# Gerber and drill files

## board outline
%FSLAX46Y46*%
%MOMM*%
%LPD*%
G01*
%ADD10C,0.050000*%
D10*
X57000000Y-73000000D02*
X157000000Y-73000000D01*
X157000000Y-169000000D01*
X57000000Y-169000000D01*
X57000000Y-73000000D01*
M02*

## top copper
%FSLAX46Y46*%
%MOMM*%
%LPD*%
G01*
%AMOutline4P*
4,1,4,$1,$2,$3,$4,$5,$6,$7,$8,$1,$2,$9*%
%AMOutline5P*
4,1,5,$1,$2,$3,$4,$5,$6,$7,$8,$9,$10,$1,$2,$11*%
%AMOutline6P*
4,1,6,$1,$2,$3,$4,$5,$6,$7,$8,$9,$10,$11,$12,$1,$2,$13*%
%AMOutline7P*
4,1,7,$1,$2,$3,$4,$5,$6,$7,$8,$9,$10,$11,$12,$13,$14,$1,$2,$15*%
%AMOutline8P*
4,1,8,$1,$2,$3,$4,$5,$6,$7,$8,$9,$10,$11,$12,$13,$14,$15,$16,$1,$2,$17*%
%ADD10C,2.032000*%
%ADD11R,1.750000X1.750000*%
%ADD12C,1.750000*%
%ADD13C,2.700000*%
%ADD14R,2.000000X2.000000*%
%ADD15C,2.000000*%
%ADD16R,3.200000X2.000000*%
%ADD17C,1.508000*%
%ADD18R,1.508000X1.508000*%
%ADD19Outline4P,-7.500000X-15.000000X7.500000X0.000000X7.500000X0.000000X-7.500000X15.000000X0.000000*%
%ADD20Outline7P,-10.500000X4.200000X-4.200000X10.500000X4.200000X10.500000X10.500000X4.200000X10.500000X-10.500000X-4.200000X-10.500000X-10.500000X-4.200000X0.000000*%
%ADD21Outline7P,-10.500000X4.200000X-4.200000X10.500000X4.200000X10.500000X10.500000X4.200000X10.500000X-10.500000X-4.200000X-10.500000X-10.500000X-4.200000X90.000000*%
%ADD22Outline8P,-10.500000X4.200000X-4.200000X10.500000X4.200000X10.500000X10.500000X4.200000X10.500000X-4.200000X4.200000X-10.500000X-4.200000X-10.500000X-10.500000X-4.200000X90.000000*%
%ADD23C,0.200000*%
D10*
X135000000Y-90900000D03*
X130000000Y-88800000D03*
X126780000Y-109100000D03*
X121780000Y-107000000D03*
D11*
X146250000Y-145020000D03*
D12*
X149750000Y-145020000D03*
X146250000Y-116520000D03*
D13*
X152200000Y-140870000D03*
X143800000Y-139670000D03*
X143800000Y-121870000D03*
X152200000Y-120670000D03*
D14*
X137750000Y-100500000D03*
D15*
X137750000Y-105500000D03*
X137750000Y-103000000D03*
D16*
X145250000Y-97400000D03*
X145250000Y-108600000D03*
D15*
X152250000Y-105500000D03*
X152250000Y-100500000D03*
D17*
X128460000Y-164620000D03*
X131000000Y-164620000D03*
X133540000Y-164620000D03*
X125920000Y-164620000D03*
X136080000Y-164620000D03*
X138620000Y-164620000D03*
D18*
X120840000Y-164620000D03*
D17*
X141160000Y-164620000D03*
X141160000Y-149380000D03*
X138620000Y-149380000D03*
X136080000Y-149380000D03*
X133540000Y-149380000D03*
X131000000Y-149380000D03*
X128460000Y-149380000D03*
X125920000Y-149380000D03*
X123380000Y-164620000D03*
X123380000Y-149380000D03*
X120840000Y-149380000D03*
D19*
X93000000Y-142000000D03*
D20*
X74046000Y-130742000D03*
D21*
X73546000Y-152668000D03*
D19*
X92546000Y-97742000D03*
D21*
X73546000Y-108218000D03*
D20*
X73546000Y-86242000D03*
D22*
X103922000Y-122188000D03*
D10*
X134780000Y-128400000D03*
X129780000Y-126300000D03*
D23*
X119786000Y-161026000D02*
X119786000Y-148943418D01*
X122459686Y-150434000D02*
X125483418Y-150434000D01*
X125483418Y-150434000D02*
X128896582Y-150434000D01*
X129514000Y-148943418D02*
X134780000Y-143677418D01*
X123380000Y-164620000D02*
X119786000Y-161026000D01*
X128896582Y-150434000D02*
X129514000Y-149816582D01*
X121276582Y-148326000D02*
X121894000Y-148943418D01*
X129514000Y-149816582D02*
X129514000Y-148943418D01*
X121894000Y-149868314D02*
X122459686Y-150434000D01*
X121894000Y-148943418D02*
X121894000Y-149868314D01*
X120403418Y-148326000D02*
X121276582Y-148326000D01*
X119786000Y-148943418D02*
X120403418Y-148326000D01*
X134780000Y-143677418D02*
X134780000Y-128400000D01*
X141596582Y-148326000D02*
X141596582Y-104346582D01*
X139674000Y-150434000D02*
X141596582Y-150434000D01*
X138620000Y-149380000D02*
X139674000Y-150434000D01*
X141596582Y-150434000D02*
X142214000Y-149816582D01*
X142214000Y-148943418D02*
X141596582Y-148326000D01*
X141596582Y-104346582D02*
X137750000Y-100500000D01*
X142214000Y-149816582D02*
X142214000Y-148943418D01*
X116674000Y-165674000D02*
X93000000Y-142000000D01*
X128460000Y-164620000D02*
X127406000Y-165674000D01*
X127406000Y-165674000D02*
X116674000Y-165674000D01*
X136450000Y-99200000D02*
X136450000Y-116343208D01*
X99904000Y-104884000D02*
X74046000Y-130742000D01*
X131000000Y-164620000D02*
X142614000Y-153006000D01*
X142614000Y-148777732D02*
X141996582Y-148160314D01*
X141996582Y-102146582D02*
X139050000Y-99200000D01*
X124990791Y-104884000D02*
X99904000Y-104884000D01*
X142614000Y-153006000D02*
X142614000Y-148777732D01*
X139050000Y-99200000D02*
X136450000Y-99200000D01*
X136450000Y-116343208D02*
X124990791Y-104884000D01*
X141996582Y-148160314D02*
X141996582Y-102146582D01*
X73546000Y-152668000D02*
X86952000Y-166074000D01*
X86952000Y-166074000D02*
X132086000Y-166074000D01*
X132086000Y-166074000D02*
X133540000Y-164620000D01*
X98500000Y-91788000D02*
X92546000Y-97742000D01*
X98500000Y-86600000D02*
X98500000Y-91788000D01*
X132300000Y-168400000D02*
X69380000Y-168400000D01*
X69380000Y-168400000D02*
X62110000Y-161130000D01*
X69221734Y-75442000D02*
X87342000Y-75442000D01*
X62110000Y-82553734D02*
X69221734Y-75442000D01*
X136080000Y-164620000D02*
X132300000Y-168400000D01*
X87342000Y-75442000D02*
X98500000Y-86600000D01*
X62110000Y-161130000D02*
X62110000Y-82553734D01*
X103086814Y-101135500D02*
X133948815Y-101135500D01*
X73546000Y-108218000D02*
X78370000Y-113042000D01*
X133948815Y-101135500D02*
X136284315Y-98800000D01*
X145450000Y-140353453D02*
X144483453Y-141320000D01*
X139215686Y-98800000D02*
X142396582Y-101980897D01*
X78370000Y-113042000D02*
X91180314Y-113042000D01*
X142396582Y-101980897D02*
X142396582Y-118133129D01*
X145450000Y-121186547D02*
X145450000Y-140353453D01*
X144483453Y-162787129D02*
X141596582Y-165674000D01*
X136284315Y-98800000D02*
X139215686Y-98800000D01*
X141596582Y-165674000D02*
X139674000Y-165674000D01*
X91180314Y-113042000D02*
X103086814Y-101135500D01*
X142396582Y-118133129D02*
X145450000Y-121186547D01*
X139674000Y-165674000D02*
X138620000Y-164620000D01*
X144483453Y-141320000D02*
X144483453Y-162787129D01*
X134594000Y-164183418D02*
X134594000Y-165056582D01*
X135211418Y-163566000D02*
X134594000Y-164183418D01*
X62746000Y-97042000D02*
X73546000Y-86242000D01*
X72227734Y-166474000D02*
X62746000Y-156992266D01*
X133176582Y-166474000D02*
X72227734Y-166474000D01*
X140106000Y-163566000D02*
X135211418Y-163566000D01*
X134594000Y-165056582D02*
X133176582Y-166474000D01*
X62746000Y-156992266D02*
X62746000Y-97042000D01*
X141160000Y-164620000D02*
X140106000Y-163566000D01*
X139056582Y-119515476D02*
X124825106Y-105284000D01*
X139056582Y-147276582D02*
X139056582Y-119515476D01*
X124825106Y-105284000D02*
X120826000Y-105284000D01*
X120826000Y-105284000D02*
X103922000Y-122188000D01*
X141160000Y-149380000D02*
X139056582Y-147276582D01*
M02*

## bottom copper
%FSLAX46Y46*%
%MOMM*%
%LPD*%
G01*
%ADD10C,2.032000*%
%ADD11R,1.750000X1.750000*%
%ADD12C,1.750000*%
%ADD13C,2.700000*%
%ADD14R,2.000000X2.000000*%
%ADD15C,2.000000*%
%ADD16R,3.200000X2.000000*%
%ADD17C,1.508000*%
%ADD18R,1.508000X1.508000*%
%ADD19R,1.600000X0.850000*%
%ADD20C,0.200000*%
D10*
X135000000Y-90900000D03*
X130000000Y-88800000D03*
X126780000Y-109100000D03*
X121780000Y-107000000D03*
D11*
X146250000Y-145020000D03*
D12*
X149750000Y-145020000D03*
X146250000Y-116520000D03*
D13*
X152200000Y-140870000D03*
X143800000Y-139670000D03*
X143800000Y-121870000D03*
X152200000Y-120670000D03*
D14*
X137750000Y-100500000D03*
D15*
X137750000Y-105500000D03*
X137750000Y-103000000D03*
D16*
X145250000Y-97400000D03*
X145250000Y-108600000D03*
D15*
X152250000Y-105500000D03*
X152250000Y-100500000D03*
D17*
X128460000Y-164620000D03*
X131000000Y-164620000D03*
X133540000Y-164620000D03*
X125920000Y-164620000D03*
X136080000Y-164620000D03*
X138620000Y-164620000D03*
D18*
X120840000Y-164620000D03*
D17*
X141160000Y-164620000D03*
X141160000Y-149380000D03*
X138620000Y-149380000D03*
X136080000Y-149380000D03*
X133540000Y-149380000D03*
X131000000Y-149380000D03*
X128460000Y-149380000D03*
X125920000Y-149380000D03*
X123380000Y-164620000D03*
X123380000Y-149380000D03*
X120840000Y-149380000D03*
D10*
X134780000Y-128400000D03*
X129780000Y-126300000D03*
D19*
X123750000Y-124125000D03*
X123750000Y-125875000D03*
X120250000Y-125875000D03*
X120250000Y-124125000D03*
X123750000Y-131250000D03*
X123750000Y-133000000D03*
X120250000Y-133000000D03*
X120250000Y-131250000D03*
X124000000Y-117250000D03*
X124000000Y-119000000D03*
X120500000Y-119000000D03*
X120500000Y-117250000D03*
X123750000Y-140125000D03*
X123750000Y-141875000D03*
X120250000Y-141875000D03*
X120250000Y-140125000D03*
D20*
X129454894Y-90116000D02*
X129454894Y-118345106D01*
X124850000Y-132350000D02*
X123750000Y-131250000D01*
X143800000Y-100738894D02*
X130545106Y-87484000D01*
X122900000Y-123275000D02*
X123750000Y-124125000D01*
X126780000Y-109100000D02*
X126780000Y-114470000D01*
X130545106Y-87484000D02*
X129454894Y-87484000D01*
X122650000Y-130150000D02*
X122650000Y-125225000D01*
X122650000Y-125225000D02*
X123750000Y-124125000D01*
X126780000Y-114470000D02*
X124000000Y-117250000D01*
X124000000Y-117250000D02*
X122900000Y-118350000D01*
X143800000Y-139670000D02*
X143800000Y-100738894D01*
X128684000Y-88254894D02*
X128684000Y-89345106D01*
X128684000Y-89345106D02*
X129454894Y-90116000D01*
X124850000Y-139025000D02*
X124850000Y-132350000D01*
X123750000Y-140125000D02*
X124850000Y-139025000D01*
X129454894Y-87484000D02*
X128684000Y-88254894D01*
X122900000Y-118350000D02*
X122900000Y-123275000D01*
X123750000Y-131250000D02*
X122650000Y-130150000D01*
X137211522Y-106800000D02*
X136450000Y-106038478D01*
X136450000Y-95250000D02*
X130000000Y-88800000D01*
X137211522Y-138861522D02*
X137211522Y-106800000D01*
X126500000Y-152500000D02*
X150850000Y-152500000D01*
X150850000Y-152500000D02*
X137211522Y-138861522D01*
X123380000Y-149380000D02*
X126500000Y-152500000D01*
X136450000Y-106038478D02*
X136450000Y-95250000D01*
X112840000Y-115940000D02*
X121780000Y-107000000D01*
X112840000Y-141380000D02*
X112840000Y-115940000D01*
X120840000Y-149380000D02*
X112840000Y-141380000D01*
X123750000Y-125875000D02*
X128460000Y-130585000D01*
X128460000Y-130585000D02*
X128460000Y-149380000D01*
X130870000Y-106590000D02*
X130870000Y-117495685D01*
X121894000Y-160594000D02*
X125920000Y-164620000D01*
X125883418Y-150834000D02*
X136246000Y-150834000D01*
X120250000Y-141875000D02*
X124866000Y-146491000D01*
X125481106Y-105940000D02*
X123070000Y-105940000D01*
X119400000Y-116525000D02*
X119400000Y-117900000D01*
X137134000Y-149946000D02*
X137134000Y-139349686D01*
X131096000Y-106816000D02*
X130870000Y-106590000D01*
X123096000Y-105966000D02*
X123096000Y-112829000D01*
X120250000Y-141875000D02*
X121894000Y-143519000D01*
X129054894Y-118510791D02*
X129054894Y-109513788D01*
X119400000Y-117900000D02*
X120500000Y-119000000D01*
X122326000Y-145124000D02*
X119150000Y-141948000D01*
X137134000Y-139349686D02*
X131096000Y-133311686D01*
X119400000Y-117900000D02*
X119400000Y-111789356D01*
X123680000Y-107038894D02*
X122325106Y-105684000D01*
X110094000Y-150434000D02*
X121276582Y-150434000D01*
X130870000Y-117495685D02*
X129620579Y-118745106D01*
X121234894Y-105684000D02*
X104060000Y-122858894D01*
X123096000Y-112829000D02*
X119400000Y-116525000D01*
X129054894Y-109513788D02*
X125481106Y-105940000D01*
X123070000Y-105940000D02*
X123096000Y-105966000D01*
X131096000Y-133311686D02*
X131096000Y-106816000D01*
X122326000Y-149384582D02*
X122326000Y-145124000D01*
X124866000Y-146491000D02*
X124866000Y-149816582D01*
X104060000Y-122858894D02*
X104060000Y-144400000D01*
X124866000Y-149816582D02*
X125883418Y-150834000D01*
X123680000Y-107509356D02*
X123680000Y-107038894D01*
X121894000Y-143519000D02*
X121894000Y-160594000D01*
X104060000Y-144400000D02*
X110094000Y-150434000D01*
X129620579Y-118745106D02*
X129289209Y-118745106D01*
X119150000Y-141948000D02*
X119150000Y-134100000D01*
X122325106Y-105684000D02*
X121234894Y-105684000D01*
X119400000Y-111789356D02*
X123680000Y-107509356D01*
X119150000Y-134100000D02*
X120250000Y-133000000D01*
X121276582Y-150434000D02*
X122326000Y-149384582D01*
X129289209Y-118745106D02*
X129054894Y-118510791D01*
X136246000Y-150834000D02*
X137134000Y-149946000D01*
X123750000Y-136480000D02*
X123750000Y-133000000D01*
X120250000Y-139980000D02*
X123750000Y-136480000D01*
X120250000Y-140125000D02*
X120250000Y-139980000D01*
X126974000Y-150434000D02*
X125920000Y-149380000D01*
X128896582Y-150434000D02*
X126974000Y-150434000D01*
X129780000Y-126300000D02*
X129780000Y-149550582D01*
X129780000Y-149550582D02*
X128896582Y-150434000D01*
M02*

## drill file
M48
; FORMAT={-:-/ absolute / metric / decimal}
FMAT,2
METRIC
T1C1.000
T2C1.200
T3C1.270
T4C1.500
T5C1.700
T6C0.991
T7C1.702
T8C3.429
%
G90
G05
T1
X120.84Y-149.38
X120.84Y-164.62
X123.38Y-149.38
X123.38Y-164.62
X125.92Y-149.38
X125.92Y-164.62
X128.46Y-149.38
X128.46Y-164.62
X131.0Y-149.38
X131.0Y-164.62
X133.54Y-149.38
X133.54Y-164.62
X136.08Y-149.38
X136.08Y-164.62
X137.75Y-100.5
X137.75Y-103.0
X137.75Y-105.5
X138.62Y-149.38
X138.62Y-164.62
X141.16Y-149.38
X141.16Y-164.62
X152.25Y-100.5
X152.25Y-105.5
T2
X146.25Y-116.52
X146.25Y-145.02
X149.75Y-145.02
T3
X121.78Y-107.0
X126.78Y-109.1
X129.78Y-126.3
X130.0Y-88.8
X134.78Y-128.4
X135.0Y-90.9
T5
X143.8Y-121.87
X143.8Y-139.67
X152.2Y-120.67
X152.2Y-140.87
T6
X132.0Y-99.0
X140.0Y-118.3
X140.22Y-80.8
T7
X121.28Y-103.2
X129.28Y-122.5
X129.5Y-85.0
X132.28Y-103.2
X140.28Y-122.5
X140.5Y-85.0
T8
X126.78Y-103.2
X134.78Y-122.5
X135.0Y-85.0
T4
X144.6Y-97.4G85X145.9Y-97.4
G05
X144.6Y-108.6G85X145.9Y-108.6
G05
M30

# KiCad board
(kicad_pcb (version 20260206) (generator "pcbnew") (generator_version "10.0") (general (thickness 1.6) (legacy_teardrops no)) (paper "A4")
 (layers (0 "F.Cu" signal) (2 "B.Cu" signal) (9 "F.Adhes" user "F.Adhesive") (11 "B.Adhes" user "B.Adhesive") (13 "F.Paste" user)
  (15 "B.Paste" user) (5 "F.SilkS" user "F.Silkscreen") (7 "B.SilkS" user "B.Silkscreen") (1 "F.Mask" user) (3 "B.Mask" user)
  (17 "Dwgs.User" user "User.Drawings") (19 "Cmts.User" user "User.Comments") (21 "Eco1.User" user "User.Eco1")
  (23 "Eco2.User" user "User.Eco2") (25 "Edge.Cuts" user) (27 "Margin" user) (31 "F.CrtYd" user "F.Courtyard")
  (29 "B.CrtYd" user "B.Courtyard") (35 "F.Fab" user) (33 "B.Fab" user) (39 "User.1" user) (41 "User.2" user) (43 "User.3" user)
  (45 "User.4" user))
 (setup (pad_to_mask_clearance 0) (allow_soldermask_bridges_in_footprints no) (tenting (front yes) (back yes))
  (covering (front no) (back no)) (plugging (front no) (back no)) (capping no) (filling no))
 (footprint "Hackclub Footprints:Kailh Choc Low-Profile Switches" (layer "F.Cu") (at 135 85)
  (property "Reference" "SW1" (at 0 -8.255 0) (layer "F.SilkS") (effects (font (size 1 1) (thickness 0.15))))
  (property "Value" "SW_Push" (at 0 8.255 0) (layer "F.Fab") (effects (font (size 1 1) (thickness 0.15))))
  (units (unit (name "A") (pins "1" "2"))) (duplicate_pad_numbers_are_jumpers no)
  (pad "" np_thru_hole circle (at -5.5 0) (size 1.7018 1.7018) (drill 1.7018) (layers "*.Cu" "*.Mask"))
  (pad "" np_thru_hole circle (at 0 0) (size 3.429 3.429) (drill 3.429) (layers "*.Cu" "*.Mask"))
  (pad "" np_thru_hole circle (at 5.22 -4.2) (size 0.9906 0.9906) (drill 0.9906) (layers "*.Cu" "*.Mask"))
  (pad "" np_thru_hole circle (at 5.5 0) (size 1.7018 1.7018) (drill 1.7018) (layers "*.Cu" "*.Mask"))
  (pad "1" thru_hole circle (at 0 5.9) (size 2.032 2.032) (drill 1.27) (layers "*.Cu" "*.Mask") (remove_unused_layers no) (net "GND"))
  (pad "2" thru_hole circle (at -5 3.8) (size 2.032 2.032) (drill 1.27) (layers "*.Cu" "*.Mask") (remove_unused_layers no) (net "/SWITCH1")))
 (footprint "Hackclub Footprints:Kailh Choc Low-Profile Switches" (layer "F.Cu") (at 126.78 103.2)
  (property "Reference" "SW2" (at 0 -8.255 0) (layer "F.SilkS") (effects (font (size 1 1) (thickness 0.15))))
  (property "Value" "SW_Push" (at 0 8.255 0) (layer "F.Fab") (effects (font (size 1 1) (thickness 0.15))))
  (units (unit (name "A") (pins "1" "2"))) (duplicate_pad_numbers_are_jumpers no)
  (pad "" np_thru_hole circle (at -5.5 0) (size 1.7018 1.7018) (drill 1.7018) (layers "*.Cu" "*.Mask"))
  (pad "" np_thru_hole circle (at 0 0) (size 3.429 3.429) (drill 3.429) (layers "*.Cu" "*.Mask"))
  (pad "" np_thru_hole circle (at 5.22 -4.2) (size 0.9906 0.9906) (drill 0.9906) (layers "*.Cu" "*.Mask"))
  (pad "" np_thru_hole circle (at 5.5 0) (size 1.7018 1.7018) (drill 1.7018) (layers "*.Cu" "*.Mask"))
  (pad "1" thru_hole circle (at 0 5.9) (size 2.032 2.032) (drill 1.27) (layers "*.Cu" "*.Mask") (remove_unused_layers no) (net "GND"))
  (pad "2" thru_hole circle (at -5 3.8) (size 2.032 2.032) (drill 1.27) (layers "*.Cu" "*.Mask") (remove_unused_layers no) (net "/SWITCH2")))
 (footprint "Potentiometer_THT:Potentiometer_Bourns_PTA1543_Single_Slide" (layer "F.Cu") (at 146.25 145.02 90)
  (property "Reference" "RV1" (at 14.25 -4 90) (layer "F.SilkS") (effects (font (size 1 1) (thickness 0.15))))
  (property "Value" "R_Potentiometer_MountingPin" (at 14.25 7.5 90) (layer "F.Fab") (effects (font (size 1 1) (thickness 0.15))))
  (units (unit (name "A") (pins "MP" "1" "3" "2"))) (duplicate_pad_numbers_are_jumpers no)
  (pad "1" thru_hole rect (at 0 0 90) (size 1.75 1.75) (drill 1.2) (layers "*.Cu" "*.Mask") (remove_unused_layers no)
   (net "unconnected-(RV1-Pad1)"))
  (pad "2" thru_hole circle (at 0 3.5 90) (size 1.75 1.75) (drill 1.2) (layers "*.Cu" "*.Mask") (remove_unused_layers no) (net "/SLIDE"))
  (pad "3" thru_hole circle (at 28.5 0 90) (size 1.75 1.75) (drill 1.2) (layers "*.Cu" "*.Mask") (remove_unused_layers no) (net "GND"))
  (pad "MP" thru_hole circle (at 4.15 5.95 90) (size 2.7 2.7) (drill 1.7) (layers "*.Cu" "*.Mask") (remove_unused_layers no) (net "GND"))
  (pad "MP" thru_hole circle (at 5.35 -2.45 90) (size 2.7 2.7) (drill 1.7) (layers "*.Cu" "*.Mask") (remove_unused_layers no) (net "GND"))
  (pad "MP" thru_hole circle (at 23.15 -2.45 90) (size 2.7 2.7) (drill 1.7) (layers "*.Cu" "*.Mask") (remove_unused_layers no) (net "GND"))
  (pad "MP" thru_hole circle (at 24.35 5.95 90) (size 2.7 2.7) (drill 1.7) (layers "*.Cu" "*.Mask") (remove_unused_layers no) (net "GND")))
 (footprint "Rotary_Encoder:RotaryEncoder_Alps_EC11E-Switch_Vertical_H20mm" (layer "F.Cu") (at 137.75 100.5)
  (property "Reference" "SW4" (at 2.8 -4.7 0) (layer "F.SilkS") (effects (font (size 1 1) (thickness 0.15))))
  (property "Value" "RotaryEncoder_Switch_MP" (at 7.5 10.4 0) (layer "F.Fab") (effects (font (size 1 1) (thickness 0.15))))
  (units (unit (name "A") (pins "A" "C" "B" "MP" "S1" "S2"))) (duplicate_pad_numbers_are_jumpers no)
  (pad "A" thru_hole rect (at 0 0) (size 2 2) (drill 1) (layers "*.Cu" "*.Mask") (remove_unused_layers no) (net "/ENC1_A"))
  (pad "B" thru_hole circle (at 0 5) (size 2 2) (drill 1) (layers "*.Cu" "*.Mask") (remove_unused_layers no) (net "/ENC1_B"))
  (pad "C" thru_hole circle (at 0 2.5) (size 2 2) (drill 1) (layers "*.Cu" "*.Mask") (remove_unused_layers no) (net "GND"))
  (pad "MP" thru_hole rect (at 7.5 -3.1) (size 3.2 2) (drill oval 2.8 1.5) (layers "*.Cu" "*.Mask") (remove_unused_layers no) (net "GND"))
  (pad "MP" thru_hole rect (at 7.5 8.1) (size 3.2 2) (drill oval 2.8 1.5) (layers "*.Cu" "*.Mask") (remove_unused_layers no) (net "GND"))
  (pad "S1" thru_hole circle (at 14.5 5) (size 2 2) (drill 1) (layers "*.Cu" "*.Mask") (remove_unused_layers no) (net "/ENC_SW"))
  (pad "S2" thru_hole circle (at 14.5 0) (size 2 2) (drill 1) (layers "*.Cu" "*.Mask") (remove_unused_layers no)
   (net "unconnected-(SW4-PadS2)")))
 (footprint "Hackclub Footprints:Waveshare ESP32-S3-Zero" (layer "F.Cu") (at 131 157 90)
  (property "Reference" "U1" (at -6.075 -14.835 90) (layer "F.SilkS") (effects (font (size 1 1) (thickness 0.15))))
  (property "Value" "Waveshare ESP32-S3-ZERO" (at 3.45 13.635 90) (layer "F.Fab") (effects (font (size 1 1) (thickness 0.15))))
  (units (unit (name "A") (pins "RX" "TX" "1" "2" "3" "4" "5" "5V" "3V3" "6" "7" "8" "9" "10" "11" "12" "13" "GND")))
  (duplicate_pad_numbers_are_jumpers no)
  (pad "1" thru_hole circle (at -7.62 -2.54 90) (size 1.508 1.508) (drill 1) (layers "*.Cu" "*.Mask") (remove_unused_layers no)
   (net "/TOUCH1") (solder_mask_margin 0.102))
  (pad "2" thru_hole circle (at -7.62 0 90) (size 1.508 1.508) (drill 1) (layers "*.Cu" "*.Mask") (remove_unused_layers no) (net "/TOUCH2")
   (solder_mask_margin 0.102))
  (pad "3" thru_hole circle (at -7.62 2.54 90) (size 1.508 1.508) (drill 1) (layers "*.Cu" "*.Mask") (remove_unused_layers no)
   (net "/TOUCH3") (solder_mask_margin 0.102))
  (pad "3V3" thru_hole circle (at -7.62 -5.08 90) (size 1.508 1.508) (drill 1) (layers "*.Cu" "*.Mask") (remove_unused_layers no)
   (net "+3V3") (solder_mask_margin 0.102))
  (pad "4" thru_hole circle (at -7.62 5.08 90) (size 1.508 1.508) (drill 1) (layers "*.Cu" "*.Mask") (remove_unused_layers no)
   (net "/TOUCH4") (solder_mask_margin 0.102))
  (pad "5" thru_hole circle (at -7.62 7.62 90) (size 1.508 1.508) (drill 1) (layers "*.Cu" "*.Mask") (remove_unused_layers no)
   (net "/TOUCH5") (solder_mask_margin 0.102))
  (pad "5V" thru_hole rect (at -7.62 -10.16 90) (size 1.508 1.508) (drill 1) (layers "*.Cu" "*.Mask") (remove_unused_layers no) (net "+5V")
   (solder_mask_margin 0.102))
  (pad "6" thru_hole circle (at -7.62 10.16 90) (size 1.508 1.508) (drill 1) (layers "*.Cu" "*.Mask") (remove_unused_layers no)
   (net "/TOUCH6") (solder_mask_margin 0.102))
  (pad "7" thru_hole circle (at 7.62 10.16 90) (size 1.508 1.508) (drill 1) (layers "*.Cu" "*.Mask") (remove_unused_layers no)
   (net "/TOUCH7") (solder_mask_margin 0.102))
  (pad "8" thru_hole circle (at 7.62 7.62 90) (size 1.508 1.508) (drill 1) (layers "*.Cu" "*.Mask") (remove_unused_layers no)
   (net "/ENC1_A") (solder_mask_margin 0.102))
  (pad "9" thru_hole circle (at 7.62 5.08 90) (size 1.508 1.508) (drill 1) (layers "*.Cu" "*.Mask") (remove_unused_layers no)
   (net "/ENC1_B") (solder_mask_margin 0.102))
  (pad "10" thru_hole circle (at 7.62 2.54 90) (size 1.508 1.508) (drill 1) (layers "*.Cu" "*.Mask") (remove_unused_layers no)
   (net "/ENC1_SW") (solder_mask_margin 0.102))
  (pad "11" thru_hole circle (at 7.62 0 90) (size 1.508 1.508) (drill 1) (layers "*.Cu" "*.Mask") (remove_unused_layers no) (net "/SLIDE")
   (solder_mask_margin 0.102))
  (pad "12" thru_hole circle (at 7.62 -2.54 90) (size 1.508 1.508) (drill 1) (layers "*.Cu" "*.Mask") (remove_unused_layers no) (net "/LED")
   (solder_mask_margin 0.102))
  (pad "13" thru_hole circle (at 7.62 -5.08 90) (size 1.508 1.508) (drill 1) (layers "*.Cu" "*.Mask") (remove_unused_layers no)
   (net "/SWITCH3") (solder_mask_margin 0.102))
  (pad "GND" thru_hole circle (at -7.62 -7.62 90) (size 1.508 1.508) (drill 1) (layers "*.Cu" "*.Mask") (remove_unused_layers no)
   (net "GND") (solder_mask_margin 0.102))
  (pad "RX" thru_hole circle (at 7.62 -7.62 90) (size 1.508 1.508) (drill 1) (layers "*.Cu" "*.Mask") (remove_unused_layers no)
   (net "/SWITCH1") (solder_mask_margin 0.102))
  (pad "TX" thru_hole circle (at 7.62 -10.16 90) (size 1.508 1.508) (drill 1) (layers "*.Cu" "*.Mask") (remove_unused_layers no)
   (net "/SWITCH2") (solder_mask_margin 0.102)))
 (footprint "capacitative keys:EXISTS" (layer "F.Cu") (at 80.046 109.742)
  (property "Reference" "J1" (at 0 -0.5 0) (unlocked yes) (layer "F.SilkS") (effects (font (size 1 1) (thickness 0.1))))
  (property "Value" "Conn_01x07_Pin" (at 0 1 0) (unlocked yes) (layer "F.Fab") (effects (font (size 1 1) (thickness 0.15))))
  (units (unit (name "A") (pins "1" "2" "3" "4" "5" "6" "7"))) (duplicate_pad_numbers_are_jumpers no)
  (pad "1" smd trapezoid (at 12.954 32.258) (size 15 15) (rect_delta 15 0) (layers "F.Cu" "F.Mask") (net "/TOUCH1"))
  (pad "2" smd roundrect (at -6 21) (size 21 21) (layers "F.Cu" "F.Mask") (roundrect_rratio 0) (chamfer_ratio 0.3)
   (chamfer top_left top_right bottom_left) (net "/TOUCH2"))
  (pad "3" smd roundrect (at -6.5 42.926 90) (size 21 21) (layers "F.Cu" "F.Mask") (roundrect_rratio 0) (chamfer_ratio 0.3)
   (chamfer top_left top_right bottom_left) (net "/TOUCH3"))
  (pad "4" smd trapezoid (at 12.5 -12) (size 15 15) (rect_delta 15 0) (layers "F.Cu" "F.Mask") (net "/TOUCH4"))
  (pad "5" smd roundrect (at -6.5 -1.524 90) (size 21 21) (layers "F.Cu" "F.Mask") (roundrect_rratio 0) (chamfer_ratio 0.3)
   (chamfer top_left top_right bottom_left) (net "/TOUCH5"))
  (pad "6" smd roundrect (at -6.5 -23.5) (size 21 21) (layers "F.Cu" "F.Mask") (roundrect_rratio 0) (chamfer_ratio 0.3)
   (chamfer top_left top_right bottom_left) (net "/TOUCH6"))
  (pad "7" smd roundrect (at 23.876 12.446 90) (size 21 21) (layers "F.Cu" "F.Mask") (roundrect_rratio 0) (chamfer_ratio 0.3)
   (chamfer top_left top_right bottom_left bottom_right) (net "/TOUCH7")))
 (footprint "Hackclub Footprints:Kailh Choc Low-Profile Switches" (layer "F.Cu") (at 134.78 122.5)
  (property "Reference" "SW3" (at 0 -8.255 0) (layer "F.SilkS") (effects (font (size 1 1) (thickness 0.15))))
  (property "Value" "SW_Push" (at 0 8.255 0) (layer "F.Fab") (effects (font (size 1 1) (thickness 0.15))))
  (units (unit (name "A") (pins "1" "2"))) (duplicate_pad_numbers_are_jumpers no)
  (pad "" np_thru_hole circle (at -5.5 0) (size 1.7018 1.7018) (drill 1.7018) (layers "*.Cu" "*.Mask"))
  (pad "" np_thru_hole circle (at 0 0) (size 3.429 3.429) (drill 3.429) (layers "*.Cu" "*.Mask"))
  (pad "" np_thru_hole circle (at 5.22 -4.2) (size 0.9906 0.9906) (drill 0.9906) (layers "*.Cu" "*.Mask"))
  (pad "" np_thru_hole circle (at 5.5 0) (size 1.7018 1.7018) (drill 1.7018) (layers "*.Cu" "*.Mask"))
  (pad "1" thru_hole circle (at 0 5.9) (size 2.032 2.032) (drill 1.27) (layers "*.Cu" "*.Mask") (remove_unused_layers no) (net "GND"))
  (pad "2" thru_hole circle (at -5 3.8) (size 2.032 2.032) (drill 1.27) (layers "*.Cu" "*.Mask") (remove_unused_layers no) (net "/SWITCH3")))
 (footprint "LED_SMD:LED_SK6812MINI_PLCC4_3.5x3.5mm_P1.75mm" (layer "B.Cu") (at 122 125 180)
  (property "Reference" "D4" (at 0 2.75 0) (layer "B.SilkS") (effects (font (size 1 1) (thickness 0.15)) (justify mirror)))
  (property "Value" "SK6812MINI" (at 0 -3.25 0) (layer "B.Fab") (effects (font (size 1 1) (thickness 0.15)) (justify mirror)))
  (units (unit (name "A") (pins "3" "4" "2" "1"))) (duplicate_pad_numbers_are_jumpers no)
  (pad "1" smd rect (at -1.75 0.875 180) (size 1.6 0.85) (layers "B.Cu" "B.Mask" "B.Paste") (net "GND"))
  (pad "2" smd rect (at -1.75 -0.875 180) (size 1.6 0.85) (layers "B.Cu" "B.Mask" "B.Paste") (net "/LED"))
  (pad "3" smd rect (at 1.75 -0.875 180) (size 1.6 0.85) (layers "B.Cu" "B.Mask" "B.Paste") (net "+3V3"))
  (pad "4" smd rect (at 1.75 0.875 180) (size 1.6 0.85) (layers "B.Cu" "B.Mask" "B.Paste") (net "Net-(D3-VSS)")))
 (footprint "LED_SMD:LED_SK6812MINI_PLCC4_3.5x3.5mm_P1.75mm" (layer "B.Cu") (at 122 132.125 180)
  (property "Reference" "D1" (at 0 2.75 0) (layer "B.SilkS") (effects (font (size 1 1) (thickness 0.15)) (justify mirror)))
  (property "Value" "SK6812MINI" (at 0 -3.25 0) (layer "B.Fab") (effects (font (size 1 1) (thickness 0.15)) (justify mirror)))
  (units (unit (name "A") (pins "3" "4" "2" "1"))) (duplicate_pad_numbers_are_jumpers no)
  (pad "1" smd rect (at -1.75 0.875 180) (size 1.6 0.85) (layers "B.Cu" "B.Mask" "B.Paste") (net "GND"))
  (pad "2" smd rect (at -1.75 -0.875 180) (size 1.6 0.85) (layers "B.Cu" "B.Mask" "B.Paste") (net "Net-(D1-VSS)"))
  (pad "3" smd rect (at 1.75 -0.875 180) (size 1.6 0.85) (layers "B.Cu" "B.Mask" "B.Paste") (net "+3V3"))
  (pad "4" smd rect (at 1.75 0.875 180) (size 1.6 0.85) (layers "B.Cu" "B.Mask" "B.Paste") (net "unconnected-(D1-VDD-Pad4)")))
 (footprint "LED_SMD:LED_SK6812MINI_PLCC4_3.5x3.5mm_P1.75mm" (layer "B.Cu") (at 122.25 118.125 180)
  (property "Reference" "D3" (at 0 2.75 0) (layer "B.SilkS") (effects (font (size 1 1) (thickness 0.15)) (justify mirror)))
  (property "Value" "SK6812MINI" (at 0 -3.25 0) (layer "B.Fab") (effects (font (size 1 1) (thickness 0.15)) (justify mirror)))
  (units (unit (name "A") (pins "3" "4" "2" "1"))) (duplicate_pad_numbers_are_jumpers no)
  (pad "1" smd rect (at -1.75 0.875 180) (size 1.6 0.85) (layers "B.Cu" "B.Mask" "B.Paste") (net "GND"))
  (pad "2" smd rect (at -1.75 -0.875 180) (size 1.6 0.85) (layers "B.Cu" "B.Mask" "B.Paste") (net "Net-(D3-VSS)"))
  (pad "3" smd rect (at 1.75 -0.875 180) (size 1.6 0.85) (layers "B.Cu" "B.Mask" "B.Paste") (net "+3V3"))
  (pad "4" smd rect (at 1.75 0.875 180) (size 1.6 0.85) (layers "B.Cu" "B.Mask" "B.Paste") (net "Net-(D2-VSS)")))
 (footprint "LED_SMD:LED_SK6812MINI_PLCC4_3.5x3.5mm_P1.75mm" (layer "B.Cu") (at 122 141 180)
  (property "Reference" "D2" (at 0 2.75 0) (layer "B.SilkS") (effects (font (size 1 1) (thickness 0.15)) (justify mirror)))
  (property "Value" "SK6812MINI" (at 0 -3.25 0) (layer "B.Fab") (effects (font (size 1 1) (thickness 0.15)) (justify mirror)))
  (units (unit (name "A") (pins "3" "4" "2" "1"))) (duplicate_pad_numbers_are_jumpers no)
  (pad "1" smd rect (at -1.75 0.875 180) (size 1.6 0.85) (layers "B.Cu" "B.Mask" "B.Paste") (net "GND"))
  (pad "2" smd rect (at -1.75 -0.875 180) (size 1.6 0.85) (layers "B.Cu" "B.Mask" "B.Paste") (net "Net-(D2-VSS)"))
  (pad "3" smd rect (at 1.75 -0.875 180) (size 1.6 0.85) (layers "B.Cu" "B.Mask" "B.Paste") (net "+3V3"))
  (pad "4" smd rect (at 1.75 0.875 180) (size 1.6 0.85) (layers "B.Cu" "B.Mask" "B.Paste") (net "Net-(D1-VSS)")))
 (gr_rect (start 57 73) (end 157 169) (stroke (width 0.05) (type default)) (fill no) (layer "Edge.Cuts"))
 (segment (start 119.786 161.026) (end 119.786 148.943418) (width 0.2) (layer "F.Cu") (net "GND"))
 (segment (start 122.459686 150.434) (end 125.483418 150.434) (width 0.2) (layer "F.Cu") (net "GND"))
 (segment (start 125.483418 150.434) (end 128.896582 150.434) (width 0.2) (layer "F.Cu") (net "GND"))
 (segment (start 129.514 148.943418) (end 134.78 143.677418) (width 0.2) (layer "F.Cu") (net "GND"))
 (segment (start 123.38 164.62) (end 119.786 161.026) (width 0.2) (layer "F.Cu") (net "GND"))
 (segment (start 128.896582 150.434) (end 129.514 149.816582) (width 0.2) (layer "F.Cu") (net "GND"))
 (segment (start 121.276582 148.326) (end 121.894 148.943418) (width 0.2) (layer "F.Cu") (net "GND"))
 (segment (start 129.514 149.816582) (end 129.514 148.943418) (width 0.2) (layer "F.Cu") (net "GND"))
 (segment (start 121.894 149.868314) (end 122.459686 150.434) (width 0.2) (layer "F.Cu") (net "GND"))
 (segment (start 121.894 148.943418) (end 121.894 149.868314) (width 0.2) (layer "F.Cu") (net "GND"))
 (segment (start 120.403418 148.326) (end 121.276582 148.326) (width 0.2) (layer "F.Cu") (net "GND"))
 (segment (start 119.786 148.943418) (end 120.403418 148.326) (width 0.2) (layer "F.Cu") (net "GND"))
 (segment (start 134.78 143.677418) (end 134.78 128.4) (width 0.2) (layer "F.Cu") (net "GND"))
 (segment (start 129.454894 90.116) (end 129.454894 118.345106) (width 0.2) (layer "B.Cu") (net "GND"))
 (segment (start 124.85 132.35) (end 123.75 131.25) (width 0.2) (layer "B.Cu") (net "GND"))
 (segment (start 143.8 100.738894) (end 130.545106 87.484) (width 0.2) (layer "B.Cu") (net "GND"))
 (segment (start 122.9 123.275) (end 123.75 124.125) (width 0.2) (layer "B.Cu") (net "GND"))
 (segment (start 126.78 109.1) (end 126.78 114.47) (width 0.2) (layer "B.Cu") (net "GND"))
 (segment (start 130.545106 87.484) (end 129.454894 87.484) (width 0.2) (layer "B.Cu") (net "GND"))
 (segment (start 122.65 130.15) (end 122.65 125.225) (width 0.2) (layer "B.Cu") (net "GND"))
 (segment (start 122.65 125.225) (end 123.75 124.125) (width 0.2) (layer "B.Cu") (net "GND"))
 (segment (start 126.78 114.47) (end 124 117.25) (width 0.2) (layer "B.Cu") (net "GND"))
 (segment (start 124 117.25) (end 122.9 118.35) (width 0.2) (layer "B.Cu") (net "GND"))
 (segment (start 143.8 139.67) (end 143.8 100.738894) (width 0.2) (layer "B.Cu") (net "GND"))
 (segment (start 128.684 88.254894) (end 128.684 89.345106) (width 0.2) (layer "B.Cu") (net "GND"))
 (segment (start 128.684 89.345106) (end 129.454894 90.116) (width 0.2) (layer "B.Cu") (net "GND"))
 (segment (start 124.85 139.025) (end 124.85 132.35) (width 0.2) (layer "B.Cu") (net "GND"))
 (segment (start 123.75 140.125) (end 124.85 139.025) (width 0.2) (layer "B.Cu") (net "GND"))
 (segment (start 129.454894 87.484) (end 128.684 88.254894) (width 0.2) (layer "B.Cu") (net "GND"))
 (segment (start 122.9 118.35) (end 122.9 123.275) (width 0.2) (layer "B.Cu") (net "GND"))
 (segment (start 123.75 131.25) (end 122.65 130.15) (width 0.2) (layer "B.Cu") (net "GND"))
 (segment (start 137.211522 106.8) (end 136.45 106.038478) (width 0.2) (layer "B.Cu") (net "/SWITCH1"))
 (segment (start 136.45 95.25) (end 130 88.8) (width 0.2) (layer "B.Cu") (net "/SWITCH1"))
 (segment (start 137.211522 138.861522) (end 137.211522 106.8) (width 0.2) (layer "B.Cu") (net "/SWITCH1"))
 (segment (start 126.5 152.5) (end 150.85 152.5) (width 0.2) (layer "B.Cu") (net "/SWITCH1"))
 (segment (start 150.85 152.5) (end 137.211522 138.861522) (width 0.2) (layer "B.Cu") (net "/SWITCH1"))
 (segment (start 123.38 149.38) (end 126.5 152.5) (width 0.2) (layer "B.Cu") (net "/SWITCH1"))
 (segment (start 136.45 106.038478) (end 136.45 95.25) (width 0.2) (layer "B.Cu") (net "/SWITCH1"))
 (segment (start 112.84 115.94) (end 121.78 107) (width 0.2) (layer "B.Cu") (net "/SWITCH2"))
 (segment (start 112.84 141.38) (end 112.84 115.94) (width 0.2) (layer "B.Cu") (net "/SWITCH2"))
 (segment (start 120.84 149.38) (end 112.84 141.38) (width 0.2) (layer "B.Cu") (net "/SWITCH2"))
 (segment (start 123.75 125.875) (end 128.46 130.585) (width 0.2) (layer "B.Cu") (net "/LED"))
 (segment (start 128.46 130.585) (end 128.46 149.38) (width 0.2) (layer "B.Cu") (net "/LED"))
 (segment (start 130.87 106.59) (end 130.87 117.495685) (width 0.2) (layer "B.Cu") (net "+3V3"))
 (segment (start 121.894 160.594) (end 125.92 164.62) (width 0.2) (layer "B.Cu") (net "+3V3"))
 (segment (start 125.883418 150.834) (end 136.246 150.834) (width 0.2) (layer "B.Cu") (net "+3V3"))
 (segment (start 120.25 141.875) (end 124.866 146.491) (width 0.2) (layer "B.Cu") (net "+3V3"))
 (segment (start 125.481106 105.94) (end 123.07 105.94) (width 0.2) (layer "B.Cu") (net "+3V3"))
 (segment (start 119.4 116.525) (end 119.4 117.9) (width 0.2) (layer "B.Cu") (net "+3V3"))
 (segment (start 137.134 149.946) (end 137.134 139.349686) (width 0.2) (layer "B.Cu") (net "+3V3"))
 (segment (start 131.096 106.816) (end 130.87 106.59) (width 0.2) (layer "B.Cu") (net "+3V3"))
 (segment (start 123.096 105.966) (end 123.096 112.829) (width 0.2) (layer "B.Cu") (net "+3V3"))
 (segment (start 120.25 141.875) (end 121.894 143.519) (width 0.2) (layer "B.Cu") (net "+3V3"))
 (segment (start 129.054894 118.510791) (end 129.054894 109.513788) (width 0.2) (layer "B.Cu") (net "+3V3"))
 (segment (start 119.4 117.9) (end 120.5 119) (width 0.2) (layer "B.Cu") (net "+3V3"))
 (segment (start 122.326 145.124) (end 119.15 141.948) (width 0.2) (layer "B.Cu") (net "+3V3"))
 (segment (start 137.134 139.349686) (end 131.096 133.311686) (width 0.2) (layer "B.Cu") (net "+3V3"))
 (segment (start 119.4 117.9) (end 119.4 111.789356) (width 0.2) (layer "B.Cu") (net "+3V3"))
 (segment (start 123.68 107.038894) (end 122.325106 105.684) (width 0.2) (layer "B.Cu") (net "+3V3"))
 (segment (start 110.094 150.434) (end 121.276582 150.434) (width 0.2) (layer "B.Cu") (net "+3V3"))
 (segment (start 130.87 117.495685) (end 129.620579 118.745106) (width 0.2) (layer "B.Cu") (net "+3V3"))
 (segment (start 121.234894 105.684) (end 104.06 122.858894) (width 0.2) (layer "B.Cu") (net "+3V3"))
 (segment (start 123.096 112.829) (end 119.4 116.525) (width 0.2) (layer "B.Cu") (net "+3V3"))
 (segment (start 129.054894 109.513788) (end 125.481106 105.94) (width 0.2) (layer "B.Cu") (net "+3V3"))
 (segment (start 123.07 105.94) (end 123.096 105.966) (width 0.2) (layer "B.Cu") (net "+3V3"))
 (segment (start 131.096 133.311686) (end 131.096 106.816) (width 0.2) (layer "B.Cu") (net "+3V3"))
 (segment (start 122.326 149.384582) (end 122.326 145.124) (width 0.2) (layer "B.Cu") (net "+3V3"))
 (segment (start 124.866 146.491) (end 124.866 149.816582) (width 0.2) (layer "B.Cu") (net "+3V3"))
 (segment (start 104.06 122.858894) (end 104.06 144.4) (width 0.2) (layer "B.Cu") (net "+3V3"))
 (segment (start 124.866 149.816582) (end 125.883418 150.834) (width 0.2) (layer "B.Cu") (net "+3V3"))
 (segment (start 123.68 107.509356) (end 123.68 107.038894) (width 0.2) (layer "B.Cu") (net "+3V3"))
 (segment (start 121.894 143.519) (end 121.894 160.594) (width 0.2) (layer "B.Cu") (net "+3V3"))
 (segment (start 104.06 144.4) (end 110.094 150.434) (width 0.2) (layer "B.Cu") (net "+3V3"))
 (segment (start 129.620579 118.745106) (end 129.289209 118.745106) (width 0.2) (layer "B.Cu") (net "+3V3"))
 (segment (start 119.15 141.948) (end 119.15 134.1) (width 0.2) (layer "B.Cu") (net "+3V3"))
 (segment (start 122.325106 105.684) (end 121.234894 105.684) (width 0.2) (layer "B.Cu") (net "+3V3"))
 (segment (start 119.4 111.789356) (end 123.68 107.509356) (width 0.2) (layer "B.Cu") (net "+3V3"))
 (segment (start 119.15 134.1) (end 120.25 133) (width 0.2) (layer "B.Cu") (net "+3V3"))
 (segment (start 121.276582 150.434) (end 122.326 149.384582) (width 0.2) (layer "B.Cu") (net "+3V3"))
 (segment (start 129.289209 118.745106) (end 129.054894 118.510791) (width 0.2) (layer "B.Cu") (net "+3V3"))
 (segment (start 136.246 150.834) (end 137.134 149.946) (width 0.2) (layer "B.Cu") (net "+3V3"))
 (segment (start 141.596582 148.326) (end 141.596582 104.346582) (width 0.2) (layer "F.Cu") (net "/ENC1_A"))
 (segment (start 139.674 150.434) (end 141.596582 150.434) (width 0.2) (layer "F.Cu") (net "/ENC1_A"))
 (segment (start 138.62 149.38) (end 139.674 150.434) (width 0.2) (layer "F.Cu") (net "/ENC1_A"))
 (segment (start 141.596582 150.434) (end 142.214 149.816582) (width 0.2) (layer "F.Cu") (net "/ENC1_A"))
 (segment (start 142.214 148.943418) (end 141.596582 148.326) (width 0.2) (layer "F.Cu") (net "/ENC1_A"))
 (segment (start 141.596582 104.346582) (end 137.75 100.5) (width 0.2) (layer "F.Cu") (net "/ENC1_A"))
 (segment (start 142.214 149.816582) (end 142.214 148.943418) (width 0.2) (layer "F.Cu") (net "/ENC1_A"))
 (segment (start 123.75 136.48) (end 123.75 133) (width 0.2) (layer "B.Cu") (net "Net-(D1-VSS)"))
 (segment (start 120.25 139.98) (end 123.75 136.48) (width 0.2) (layer "B.Cu") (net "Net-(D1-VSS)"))
 (segment (start 120.25 140.125) (end 120.25 139.98) (width 0.2) (layer "B.Cu") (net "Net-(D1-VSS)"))
 (segment (start 116.674 165.674) (end 93 142) (width 0.2) (layer "F.Cu") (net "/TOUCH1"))
 (segment (start 128.46 164.62) (end 127.406 165.674) (width 0.2) (layer "F.Cu") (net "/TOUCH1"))
 (segment (start 127.406 165.674) (end 116.674 165.674) (width 0.2) (layer "F.Cu") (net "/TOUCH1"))
 (segment (start 136.45 99.2) (end 136.45 116.343208) (width 0.2) (layer "F.Cu") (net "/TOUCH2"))
 (segment (start 99.904 104.884) (end 74.046 130.742) (width 0.2) (layer "F.Cu") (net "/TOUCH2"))
 (segment (start 131 164.62) (end 142.614 153.006) (width 0.2) (layer "F.Cu") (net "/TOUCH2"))
 (segment (start 142.614 148.777732) (end 141.996582 148.160314) (width 0.2) (layer "F.Cu") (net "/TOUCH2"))
 (segment (start 141.996582 102.146582) (end 139.05 99.2) (width 0.2) (layer "F.Cu") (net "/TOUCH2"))
 (segment (start 124.990791 104.884) (end 99.904 104.884) (width 0.2) (layer "F.Cu") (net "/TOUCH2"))
 (segment (start 142.614 153.006) (end 142.614 148.777732) (width 0.2) (layer "F.Cu") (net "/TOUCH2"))
 (segment (start 139.05 99.2) (end 136.45 99.2) (width 0.2) (layer "F.Cu") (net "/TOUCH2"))
 (segment (start 136.45 116.343208) (end 124.990791 104.884) (width 0.2) (layer "F.Cu") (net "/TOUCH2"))
 (segment (start 141.996582 148.160314) (end 141.996582 102.146582) (width 0.2) (layer "F.Cu") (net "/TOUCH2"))
 (segment (start 73.546 152.668) (end 86.952 166.074) (width 0.2) (layer "F.Cu") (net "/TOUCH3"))
 (segment (start 86.952 166.074) (end 132.086 166.074) (width 0.2) (layer "F.Cu") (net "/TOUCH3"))
 (segment (start 132.086 166.074) (end 133.54 164.62) (width 0.2) (layer "F.Cu") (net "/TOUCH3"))
 (segment (start 98.5 91.788) (end 92.546 97.742) (width 0.2) (layer "F.Cu") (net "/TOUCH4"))
 (segment (start 98.5 86.6) (end 98.5 91.788) (width 0.2) (layer "F.Cu") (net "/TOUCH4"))
 (segment (start 132.3 168.4) (end 69.38 168.4) (width 0.2) (layer "F.Cu") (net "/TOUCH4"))
 (segment (start 69.38 168.4) (end 62.11 161.13) (width 0.2) (layer "F.Cu") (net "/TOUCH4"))
 (segment (start 69.221734 75.442) (end 87.342 75.442) (width 0.2) (layer "F.Cu") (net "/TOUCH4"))
 (segment (start 62.11 82.553734) (end 69.221734 75.442) (width 0.2) (layer "F.Cu") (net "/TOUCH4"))
 (segment (start 136.08 164.62) (end 132.3 168.4) (width 0.2) (layer "F.Cu") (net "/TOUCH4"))
 (segment (start 87.342 75.442) (end 98.5 86.6) (width 0.2) (layer "F.Cu") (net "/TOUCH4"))
 (segment (start 62.11 161.13) (end 62.11 82.553734) (width 0.2) (layer "F.Cu") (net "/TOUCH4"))
 (segment (start 103.086814 101.1355) (end 133.948815 101.1355) (width 0.2) (layer "F.Cu") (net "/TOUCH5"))
 (segment (start 73.546 108.218) (end 78.37 113.042) (width 0.2) (layer "F.Cu") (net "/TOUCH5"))
 (segment (start 133.948815 101.1355) (end 136.284315 98.8) (width 0.2) (layer "F.Cu") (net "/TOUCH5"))
 (segment (start 145.45 140.353453) (end 144.483453 141.32) (width 0.2) (layer "F.Cu") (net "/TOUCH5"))
 (segment (start 139.215686 98.8) (end 142.396582 101.980897) (width 0.2) (layer "F.Cu") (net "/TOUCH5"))
 (segment (start 78.37 113.042) (end 91.180314 113.042) (width 0.2) (layer "F.Cu") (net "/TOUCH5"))
 (segment (start 142.396582 101.980897) (end 142.396582 118.133129) (width 0.2) (layer "F.Cu") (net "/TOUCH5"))
 (segment (start 145.45 121.186547) (end 145.45 140.353453) (width 0.2) (layer "F.Cu") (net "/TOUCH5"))
 (segment (start 144.483453 162.787129) (end 141.596582 165.674) (width 0.2) (layer "F.Cu") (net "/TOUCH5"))
 (segment (start 136.284315 98.8) (end 139.215686 98.8) (width 0.2) (layer "F.Cu") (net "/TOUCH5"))
 (segment (start 141.596582 165.674) (end 139.674 165.674) (width 0.2) (layer "F.Cu") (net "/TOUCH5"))
 (segment (start 91.180314 113.042) (end 103.086814 101.1355) (width 0.2) (layer "F.Cu") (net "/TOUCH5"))
 (segment (start 142.396582 118.133129) (end 145.45 121.186547) (width 0.2) (layer "F.Cu") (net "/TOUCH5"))
 (segment (start 139.674 165.674) (end 138.62 164.62) (width 0.2) (layer "F.Cu") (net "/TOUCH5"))
 (segment (start 144.483453 141.32) (end 144.483453 162.787129) (width 0.2) (layer "F.Cu") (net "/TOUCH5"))
 (segment (start 134.594 164.183418) (end 134.594 165.056582) (width 0.2) (layer "F.Cu") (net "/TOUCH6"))
 (segment (start 135.211418 163.566) (end 134.594 164.183418) (width 0.2) (layer "F.Cu") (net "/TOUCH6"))
 (segment (start 62.746 97.042) (end 73.546 86.242) (width 0.2) (layer "F.Cu") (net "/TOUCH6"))
 (segment (start 72.227734 166.474) (end 62.746 156.992266) (width 0.2) (layer "F.Cu") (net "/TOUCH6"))
 (segment (start 133.176582 166.474) (end 72.227734 166.474) (width 0.2) (layer "F.Cu") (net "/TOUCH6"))
 (segment (start 140.106 163.566) (end 135.211418 163.566) (width 0.2) (layer "F.Cu") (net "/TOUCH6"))
 (segment (start 134.594 165.056582) (end 133.176582 166.474) (width 0.2) (layer "F.Cu") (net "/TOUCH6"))
 (segment (start 62.746 156.992266) (end 62.746 97.042) (width 0.2) (layer "F.Cu") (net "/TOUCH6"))
 (segment (start 141.16 164.62) (end 140.106 163.566) (width 0.2) (layer "F.Cu") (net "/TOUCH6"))
 (segment (start 139.056582 119.515476) (end 124.825106 105.284) (width 0.2) (layer "F.Cu") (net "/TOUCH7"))
 (segment (start 139.056582 147.276582) (end 139.056582 119.515476) (width 0.2) (layer "F.Cu") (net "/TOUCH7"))
 (segment (start 124.825106 105.284) (end 120.826 105.284) (width 0.2) (layer "F.Cu") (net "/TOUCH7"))
 (segment (start 120.826 105.284) (end 103.922 122.188) (width 0.2) (layer "F.Cu") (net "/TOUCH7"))
 (segment (start 141.16 149.38) (end 139.056582 147.276582) (width 0.2) (layer "F.Cu") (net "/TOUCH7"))
 (segment (start 126.974 150.434) (end 125.92 149.38) (width 0.2) (layer "B.Cu") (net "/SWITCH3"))
 (segment (start 128.896582 150.434) (end 126.974 150.434) (width 0.2) (layer "B.Cu") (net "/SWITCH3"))
 (segment (start 129.78 126.3) (end 129.78 149.550582) (width 0.2) (layer "B.Cu") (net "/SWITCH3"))
 (segment (start 129.78 149.550582) (end 128.896582 150.434) (width 0.2) (layer "B.Cu") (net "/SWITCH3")))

